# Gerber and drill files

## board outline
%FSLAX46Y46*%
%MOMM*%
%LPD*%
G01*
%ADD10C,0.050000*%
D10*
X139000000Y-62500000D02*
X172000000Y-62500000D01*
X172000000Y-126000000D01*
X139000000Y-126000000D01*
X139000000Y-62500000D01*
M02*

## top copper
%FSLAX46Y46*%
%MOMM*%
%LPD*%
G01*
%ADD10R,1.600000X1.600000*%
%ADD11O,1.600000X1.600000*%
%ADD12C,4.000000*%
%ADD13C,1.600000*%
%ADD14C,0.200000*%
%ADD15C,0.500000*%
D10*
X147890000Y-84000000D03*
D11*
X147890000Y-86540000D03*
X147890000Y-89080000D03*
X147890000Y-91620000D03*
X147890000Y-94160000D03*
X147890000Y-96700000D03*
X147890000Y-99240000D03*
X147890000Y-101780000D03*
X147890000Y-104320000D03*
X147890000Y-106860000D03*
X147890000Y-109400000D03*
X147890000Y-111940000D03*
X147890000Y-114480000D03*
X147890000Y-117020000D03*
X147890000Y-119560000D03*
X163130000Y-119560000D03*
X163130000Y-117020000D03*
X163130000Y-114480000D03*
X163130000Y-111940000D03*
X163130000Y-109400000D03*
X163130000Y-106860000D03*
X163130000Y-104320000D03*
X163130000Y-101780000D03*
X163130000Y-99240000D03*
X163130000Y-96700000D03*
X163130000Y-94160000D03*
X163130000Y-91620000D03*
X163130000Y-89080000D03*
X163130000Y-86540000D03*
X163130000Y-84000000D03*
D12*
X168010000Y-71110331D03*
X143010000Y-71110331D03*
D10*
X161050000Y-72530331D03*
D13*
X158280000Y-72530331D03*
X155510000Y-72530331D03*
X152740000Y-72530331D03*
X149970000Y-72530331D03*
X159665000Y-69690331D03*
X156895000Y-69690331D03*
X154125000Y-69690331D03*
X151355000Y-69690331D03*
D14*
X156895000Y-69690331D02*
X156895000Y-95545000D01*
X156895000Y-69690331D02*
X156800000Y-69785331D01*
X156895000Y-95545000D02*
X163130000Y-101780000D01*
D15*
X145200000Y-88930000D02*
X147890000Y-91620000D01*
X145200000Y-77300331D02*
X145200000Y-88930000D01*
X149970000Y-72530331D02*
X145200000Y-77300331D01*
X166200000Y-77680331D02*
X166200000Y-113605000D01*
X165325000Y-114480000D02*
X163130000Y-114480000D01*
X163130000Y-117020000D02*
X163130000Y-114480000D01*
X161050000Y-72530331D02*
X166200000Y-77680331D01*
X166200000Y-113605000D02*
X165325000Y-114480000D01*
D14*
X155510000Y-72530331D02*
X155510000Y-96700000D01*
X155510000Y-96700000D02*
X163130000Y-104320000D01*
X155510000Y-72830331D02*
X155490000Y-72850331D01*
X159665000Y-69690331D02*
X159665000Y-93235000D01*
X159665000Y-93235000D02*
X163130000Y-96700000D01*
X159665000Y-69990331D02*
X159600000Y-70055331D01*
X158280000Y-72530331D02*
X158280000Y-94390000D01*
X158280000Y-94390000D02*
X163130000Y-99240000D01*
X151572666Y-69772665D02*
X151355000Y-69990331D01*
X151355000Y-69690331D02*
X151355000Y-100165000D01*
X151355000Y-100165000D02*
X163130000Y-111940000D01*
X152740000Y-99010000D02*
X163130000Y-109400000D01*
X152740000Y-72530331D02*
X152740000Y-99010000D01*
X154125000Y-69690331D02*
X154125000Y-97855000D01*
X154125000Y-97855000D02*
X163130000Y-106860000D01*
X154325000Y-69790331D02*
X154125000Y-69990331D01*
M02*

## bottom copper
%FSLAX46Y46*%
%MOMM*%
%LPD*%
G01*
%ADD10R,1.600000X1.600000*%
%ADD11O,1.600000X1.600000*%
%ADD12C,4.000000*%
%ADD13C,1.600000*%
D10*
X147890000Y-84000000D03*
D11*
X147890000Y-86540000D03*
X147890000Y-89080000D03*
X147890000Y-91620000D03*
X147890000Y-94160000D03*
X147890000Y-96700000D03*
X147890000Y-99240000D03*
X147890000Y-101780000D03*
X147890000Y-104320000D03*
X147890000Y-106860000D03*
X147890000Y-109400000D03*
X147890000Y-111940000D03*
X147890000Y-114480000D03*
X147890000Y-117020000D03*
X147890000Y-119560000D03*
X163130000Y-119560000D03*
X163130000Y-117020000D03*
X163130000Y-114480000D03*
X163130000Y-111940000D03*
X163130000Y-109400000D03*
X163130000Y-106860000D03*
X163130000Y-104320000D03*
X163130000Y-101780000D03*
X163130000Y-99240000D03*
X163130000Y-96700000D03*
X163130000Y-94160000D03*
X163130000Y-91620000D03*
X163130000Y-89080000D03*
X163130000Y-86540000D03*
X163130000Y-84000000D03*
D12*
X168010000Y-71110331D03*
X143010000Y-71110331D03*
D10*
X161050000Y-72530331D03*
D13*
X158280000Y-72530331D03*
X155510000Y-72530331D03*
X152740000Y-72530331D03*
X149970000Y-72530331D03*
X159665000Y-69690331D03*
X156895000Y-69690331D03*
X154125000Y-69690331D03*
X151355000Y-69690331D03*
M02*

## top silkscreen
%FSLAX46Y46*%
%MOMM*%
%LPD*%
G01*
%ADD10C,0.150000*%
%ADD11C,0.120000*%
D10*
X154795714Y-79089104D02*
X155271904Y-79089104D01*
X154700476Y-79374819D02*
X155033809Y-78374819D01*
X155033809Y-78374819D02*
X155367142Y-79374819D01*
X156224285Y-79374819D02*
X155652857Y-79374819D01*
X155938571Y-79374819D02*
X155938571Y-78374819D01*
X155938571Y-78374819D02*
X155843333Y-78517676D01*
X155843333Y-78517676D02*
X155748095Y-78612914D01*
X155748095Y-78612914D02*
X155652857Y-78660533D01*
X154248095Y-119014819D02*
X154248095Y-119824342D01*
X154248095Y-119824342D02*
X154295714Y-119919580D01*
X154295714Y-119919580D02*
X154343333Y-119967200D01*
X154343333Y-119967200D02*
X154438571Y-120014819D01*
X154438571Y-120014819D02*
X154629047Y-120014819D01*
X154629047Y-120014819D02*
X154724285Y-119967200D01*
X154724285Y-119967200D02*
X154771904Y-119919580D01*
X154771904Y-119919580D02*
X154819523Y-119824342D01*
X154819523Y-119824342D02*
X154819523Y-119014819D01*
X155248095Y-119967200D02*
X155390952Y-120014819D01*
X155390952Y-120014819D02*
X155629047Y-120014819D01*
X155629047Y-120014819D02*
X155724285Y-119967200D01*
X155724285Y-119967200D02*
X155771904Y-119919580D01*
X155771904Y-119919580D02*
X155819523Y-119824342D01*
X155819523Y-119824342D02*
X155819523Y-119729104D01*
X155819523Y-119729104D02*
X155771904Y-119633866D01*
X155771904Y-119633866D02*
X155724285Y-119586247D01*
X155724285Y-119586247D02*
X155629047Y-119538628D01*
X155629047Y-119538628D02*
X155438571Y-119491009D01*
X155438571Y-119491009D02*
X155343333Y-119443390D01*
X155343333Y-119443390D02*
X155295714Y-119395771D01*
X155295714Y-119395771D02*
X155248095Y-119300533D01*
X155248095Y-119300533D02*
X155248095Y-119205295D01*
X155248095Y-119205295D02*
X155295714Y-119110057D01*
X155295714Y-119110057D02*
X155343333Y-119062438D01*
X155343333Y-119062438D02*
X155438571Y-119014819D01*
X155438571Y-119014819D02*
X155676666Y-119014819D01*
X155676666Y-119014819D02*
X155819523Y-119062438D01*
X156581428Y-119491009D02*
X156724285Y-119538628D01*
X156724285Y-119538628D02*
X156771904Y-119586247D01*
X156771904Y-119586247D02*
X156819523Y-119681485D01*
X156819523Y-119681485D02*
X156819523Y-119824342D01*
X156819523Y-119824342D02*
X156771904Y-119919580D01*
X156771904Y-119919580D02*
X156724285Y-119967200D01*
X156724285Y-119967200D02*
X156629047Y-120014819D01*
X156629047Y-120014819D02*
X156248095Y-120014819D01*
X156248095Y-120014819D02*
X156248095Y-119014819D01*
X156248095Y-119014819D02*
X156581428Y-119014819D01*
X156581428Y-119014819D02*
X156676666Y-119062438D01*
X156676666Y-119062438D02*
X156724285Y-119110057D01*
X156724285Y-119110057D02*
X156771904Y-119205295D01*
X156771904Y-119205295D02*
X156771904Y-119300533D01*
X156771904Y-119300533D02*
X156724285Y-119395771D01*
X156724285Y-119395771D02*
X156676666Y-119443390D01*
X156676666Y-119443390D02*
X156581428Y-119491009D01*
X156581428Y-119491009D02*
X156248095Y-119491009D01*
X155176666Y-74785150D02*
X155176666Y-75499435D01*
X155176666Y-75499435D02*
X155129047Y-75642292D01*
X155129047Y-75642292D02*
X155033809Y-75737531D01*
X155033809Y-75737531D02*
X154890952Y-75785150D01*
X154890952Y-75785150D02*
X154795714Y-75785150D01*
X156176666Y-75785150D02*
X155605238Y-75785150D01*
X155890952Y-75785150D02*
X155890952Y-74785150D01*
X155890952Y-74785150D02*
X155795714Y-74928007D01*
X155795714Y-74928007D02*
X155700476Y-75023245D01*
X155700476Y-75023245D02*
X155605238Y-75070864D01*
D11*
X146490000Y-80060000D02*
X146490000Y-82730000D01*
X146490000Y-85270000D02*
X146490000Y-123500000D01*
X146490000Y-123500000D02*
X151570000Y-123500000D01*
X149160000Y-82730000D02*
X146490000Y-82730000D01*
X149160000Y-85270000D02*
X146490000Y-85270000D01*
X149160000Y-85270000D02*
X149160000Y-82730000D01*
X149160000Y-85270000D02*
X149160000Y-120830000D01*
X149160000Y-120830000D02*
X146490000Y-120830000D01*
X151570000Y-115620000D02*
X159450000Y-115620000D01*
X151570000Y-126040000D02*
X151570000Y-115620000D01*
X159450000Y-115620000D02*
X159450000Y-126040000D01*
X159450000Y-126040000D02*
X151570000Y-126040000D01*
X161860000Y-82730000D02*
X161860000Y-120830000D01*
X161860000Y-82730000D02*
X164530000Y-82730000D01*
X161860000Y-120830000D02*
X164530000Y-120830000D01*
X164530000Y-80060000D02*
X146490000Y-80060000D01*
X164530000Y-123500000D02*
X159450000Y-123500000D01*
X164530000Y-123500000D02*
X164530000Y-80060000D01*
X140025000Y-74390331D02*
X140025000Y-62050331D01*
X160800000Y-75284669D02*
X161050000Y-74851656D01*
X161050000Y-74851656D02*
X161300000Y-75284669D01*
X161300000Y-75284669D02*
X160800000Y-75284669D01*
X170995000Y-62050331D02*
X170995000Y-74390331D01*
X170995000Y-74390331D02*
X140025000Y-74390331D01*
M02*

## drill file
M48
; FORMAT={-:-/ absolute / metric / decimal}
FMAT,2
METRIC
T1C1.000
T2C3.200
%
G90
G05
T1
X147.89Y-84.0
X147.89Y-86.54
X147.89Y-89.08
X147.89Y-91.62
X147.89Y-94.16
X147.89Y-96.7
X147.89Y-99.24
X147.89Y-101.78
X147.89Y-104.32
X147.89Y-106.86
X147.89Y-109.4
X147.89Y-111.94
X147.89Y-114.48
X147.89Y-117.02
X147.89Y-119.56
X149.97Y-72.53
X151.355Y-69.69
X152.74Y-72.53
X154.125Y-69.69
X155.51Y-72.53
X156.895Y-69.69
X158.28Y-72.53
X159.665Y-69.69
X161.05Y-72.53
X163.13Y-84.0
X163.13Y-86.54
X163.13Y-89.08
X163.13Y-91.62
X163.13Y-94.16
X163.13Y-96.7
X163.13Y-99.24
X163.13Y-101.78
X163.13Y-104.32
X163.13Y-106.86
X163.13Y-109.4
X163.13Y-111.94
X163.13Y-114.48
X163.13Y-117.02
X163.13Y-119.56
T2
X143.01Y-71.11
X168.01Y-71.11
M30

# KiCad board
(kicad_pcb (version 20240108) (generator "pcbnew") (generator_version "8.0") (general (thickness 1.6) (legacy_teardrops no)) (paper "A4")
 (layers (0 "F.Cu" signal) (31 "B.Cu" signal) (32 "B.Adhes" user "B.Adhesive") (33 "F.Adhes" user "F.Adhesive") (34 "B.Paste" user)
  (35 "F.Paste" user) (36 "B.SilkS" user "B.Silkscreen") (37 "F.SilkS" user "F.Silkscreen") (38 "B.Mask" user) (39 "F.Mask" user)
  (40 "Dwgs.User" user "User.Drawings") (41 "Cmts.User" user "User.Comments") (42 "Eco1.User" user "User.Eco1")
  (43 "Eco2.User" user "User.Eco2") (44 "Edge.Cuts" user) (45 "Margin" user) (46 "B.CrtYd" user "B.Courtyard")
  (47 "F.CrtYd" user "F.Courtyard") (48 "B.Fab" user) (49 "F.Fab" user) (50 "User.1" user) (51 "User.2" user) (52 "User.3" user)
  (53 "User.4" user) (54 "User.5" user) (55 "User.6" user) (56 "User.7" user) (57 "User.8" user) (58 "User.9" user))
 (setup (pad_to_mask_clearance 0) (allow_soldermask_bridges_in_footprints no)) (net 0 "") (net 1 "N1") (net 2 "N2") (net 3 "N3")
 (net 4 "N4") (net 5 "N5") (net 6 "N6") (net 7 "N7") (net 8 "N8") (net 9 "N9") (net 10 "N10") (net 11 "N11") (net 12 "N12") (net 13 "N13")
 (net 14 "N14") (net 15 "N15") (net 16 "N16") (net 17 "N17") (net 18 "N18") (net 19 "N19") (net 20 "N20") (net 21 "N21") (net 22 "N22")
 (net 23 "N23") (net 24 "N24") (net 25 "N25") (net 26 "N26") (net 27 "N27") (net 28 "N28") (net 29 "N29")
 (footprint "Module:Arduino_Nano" (layer "F.Cu") (at 147.89 84)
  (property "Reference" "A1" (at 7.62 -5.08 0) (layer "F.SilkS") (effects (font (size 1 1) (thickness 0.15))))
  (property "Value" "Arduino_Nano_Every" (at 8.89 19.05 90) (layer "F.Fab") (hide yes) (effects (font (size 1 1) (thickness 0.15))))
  (fp_line (start -1.4 -3.94) (end -1.4 -1.27) (stroke (width 0.12) (type solid)) (layer "F.SilkS"))
  (fp_line (start -1.4 1.27) (end -1.4 39.5) (stroke (width 0.12) (type solid)) (layer "F.SilkS"))
  (fp_line (start -1.4 39.5) (end 3.68 39.5) (stroke (width 0.12) (type solid)) (layer "F.SilkS"))
  (fp_line (start 1.27 -1.27) (end -1.4 -1.27) (stroke (width 0.12) (type solid)) (layer "F.SilkS"))
  (fp_line (start 1.27 1.27) (end -1.4 1.27) (stroke (width 0.12) (type solid)) (layer "F.SilkS"))
  (fp_line (start 1.27 1.27) (end 1.27 -1.27) (stroke (width 0.12) (type solid)) (layer "F.SilkS"))
  (fp_line (start 1.27 1.27) (end 1.27 36.83) (stroke (width 0.12) (type solid)) (layer "F.SilkS"))
  (fp_line (start 1.27 36.83) (end -1.4 36.83) (stroke (width 0.12) (type solid)) (layer "F.SilkS"))
  (fp_line (start 3.68 31.62) (end 11.56 31.62) (stroke (width 0.12) (type solid)) (layer "F.SilkS"))
  (fp_line (start 3.68 42.04) (end 3.68 31.62) (stroke (width 0.12) (type solid)) (layer "F.SilkS"))
  (fp_line (start 11.56 31.62) (end 11.56 42.04) (stroke (width 0.12) (type solid)) (layer "F.SilkS"))
  (fp_line (start 11.56 42.04) (end 3.68 42.04) (stroke (width 0.12) (type solid)) (layer "F.SilkS"))
  (fp_line (start 13.97 -1.27) (end 13.97 36.83) (stroke (width 0.12) (type solid)) (layer "F.SilkS"))
  (fp_line (start 13.97 -1.27) (end 16.64 -1.27) (stroke (width 0.12) (type solid)) (layer "F.SilkS"))
  (fp_line (start 13.97 36.83) (end 16.64 36.83) (stroke (width 0.12) (type solid)) (layer "F.SilkS"))
  (fp_line (start 16.64 -3.94) (end -1.4 -3.94) (stroke (width 0.12) (type solid)) (layer "F.SilkS"))
  (fp_line (start 16.64 39.5) (end 11.56 39.5) (stroke (width 0.12) (type solid)) (layer "F.SilkS"))
  (fp_line (start 16.64 39.5) (end 16.64 -3.94) (stroke (width 0.12) (type solid)) (layer "F.SilkS"))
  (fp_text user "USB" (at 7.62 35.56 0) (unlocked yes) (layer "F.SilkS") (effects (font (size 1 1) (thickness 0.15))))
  (pad "1" thru_hole rect (at 0 0) (size 1.6 1.6) (drill 1) (layers "*.Cu" "*.Mask") (remove_unused_layers no) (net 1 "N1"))
  (pad "2" thru_hole oval (at 0 2.54) (size 1.6 1.6) (drill 1) (layers "*.Cu" "*.Mask") (remove_unused_layers no) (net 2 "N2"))
  (pad "3" thru_hole oval (at 0 5.08) (size 1.6 1.6) (drill 1) (layers "*.Cu" "*.Mask") (remove_unused_layers no) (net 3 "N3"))
  (pad "4" thru_hole oval (at 0 7.62) (size 1.6 1.6) (drill 1) (layers "*.Cu" "*.Mask") (remove_unused_layers no) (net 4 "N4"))
  (pad "5" thru_hole oval (at 0 10.16) (size 1.6 1.6) (drill 1) (layers "*.Cu" "*.Mask") (remove_unused_layers no) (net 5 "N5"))
  (pad "6" thru_hole oval (at 0 12.7) (size 1.6 1.6) (drill 1) (layers "*.Cu" "*.Mask") (remove_unused_layers no) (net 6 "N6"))
  (pad "7" thru_hole oval (at 0 15.24) (size 1.6 1.6) (drill 1) (layers "*.Cu" "*.Mask") (remove_unused_layers no) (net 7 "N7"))
  (pad "8" thru_hole oval (at 0 17.78) (size 1.6 1.6) (drill 1) (layers "*.Cu" "*.Mask") (remove_unused_layers no) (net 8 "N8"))
  (pad "9" thru_hole oval (at 0 20.32) (size 1.6 1.6) (drill 1) (layers "*.Cu" "*.Mask") (remove_unused_layers no) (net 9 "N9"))
  (pad "10" thru_hole oval (at 0 22.86) (size 1.6 1.6) (drill 1) (layers "*.Cu" "*.Mask") (remove_unused_layers no) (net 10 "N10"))
  (pad "11" thru_hole oval (at 0 25.4) (size 1.6 1.6) (drill 1) (layers "*.Cu" "*.Mask") (remove_unused_layers no) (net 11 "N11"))
  (pad "12" thru_hole oval (at 0 27.94) (size 1.6 1.6) (drill 1) (layers "*.Cu" "*.Mask") (remove_unused_layers no) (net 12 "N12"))
  (pad "13" thru_hole oval (at 0 30.48) (size 1.6 1.6) (drill 1) (layers "*.Cu" "*.Mask") (remove_unused_layers no) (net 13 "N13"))
  (pad "14" thru_hole oval (at 0 33.02) (size 1.6 1.6) (drill 1) (layers "*.Cu" "*.Mask") (remove_unused_layers no) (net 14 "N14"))
  (pad "15" thru_hole oval (at 0 35.56) (size 1.6 1.6) (drill 1) (layers "*.Cu" "*.Mask") (remove_unused_layers no) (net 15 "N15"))
  (pad "16" thru_hole oval (at 15.24 35.56) (size 1.6 1.6) (drill 1) (layers "*.Cu" "*.Mask") (remove_unused_layers no) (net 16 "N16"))
  (pad "17" thru_hole oval (at 15.24 33.02) (size 1.6 1.6) (drill 1) (layers "*.Cu" "*.Mask") (remove_unused_layers no) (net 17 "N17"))
  (pad "18" thru_hole oval (at 15.24 30.48) (size 1.6 1.6) (drill 1) (layers "*.Cu" "*.Mask") (remove_unused_layers no) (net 17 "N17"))
  (pad "19" thru_hole oval (at 15.24 27.94) (size 1.6 1.6) (drill 1) (layers "*.Cu" "*.Mask") (remove_unused_layers no) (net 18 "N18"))
  (pad "20" thru_hole oval (at 15.24 25.4) (size 1.6 1.6) (drill 1) (layers "*.Cu" "*.Mask") (remove_unused_layers no) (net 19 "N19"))
  (pad "21" thru_hole oval (at 15.24 22.86) (size 1.6 1.6) (drill 1) (layers "*.Cu" "*.Mask") (remove_unused_layers no) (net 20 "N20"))
  (pad "22" thru_hole oval (at 15.24 20.32) (size 1.6 1.6) (drill 1) (layers "*.Cu" "*.Mask") (remove_unused_layers no) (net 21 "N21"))
  (pad "23" thru_hole oval (at 15.24 17.78) (size 1.6 1.6) (drill 1) (layers "*.Cu" "*.Mask") (remove_unused_layers no) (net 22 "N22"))
  (pad "24" thru_hole oval (at 15.24 15.24) (size 1.6 1.6) (drill 1) (layers "*.Cu" "*.Mask") (remove_unused_layers no) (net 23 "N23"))
  (pad "25" thru_hole oval (at 15.24 12.7) (size 1.6 1.6) (drill 1) (layers "*.Cu" "*.Mask") (remove_unused_layers no) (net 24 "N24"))
  (pad "26" thru_hole oval (at 15.24 10.16) (size 1.6 1.6) (drill 1) (layers "*.Cu" "*.Mask") (remove_unused_layers no) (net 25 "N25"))
  (pad "27" thru_hole oval (at 15.24 7.62) (size 1.6 1.6) (drill 1) (layers "*.Cu" "*.Mask") (remove_unused_layers no) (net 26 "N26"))
  (pad "28" thru_hole oval (at 15.24 5.08) (size 1.6 1.6) (drill 1) (layers "*.Cu" "*.Mask") (remove_unused_layers no) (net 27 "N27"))
  (pad "29" thru_hole oval (at 15.24 2.54) (size 1.6 1.6) (drill 1) (layers "*.Cu" "*.Mask") (remove_unused_layers no) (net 4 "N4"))
  (pad "30" thru_hole oval (at 15.24 0) (size 1.6 1.6) (drill 1) (layers "*.Cu" "*.Mask") (remove_unused_layers no) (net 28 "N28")))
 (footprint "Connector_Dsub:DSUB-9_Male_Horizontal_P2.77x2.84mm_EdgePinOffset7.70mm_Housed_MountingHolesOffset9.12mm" (layer "F.Cu")
  (at 161.05 72.530331 180)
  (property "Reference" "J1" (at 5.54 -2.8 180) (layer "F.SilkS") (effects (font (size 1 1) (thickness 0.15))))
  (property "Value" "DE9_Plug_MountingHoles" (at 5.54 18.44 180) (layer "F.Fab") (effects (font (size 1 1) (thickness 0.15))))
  (fp_line (start 21.025 -1.86) (end 21.025 10.48) (stroke (width 0.12) (type solid)) (layer "F.SilkS"))
  (fp_line (start 0.25 -2.754338) (end 0 -2.321325) (stroke (width 0.12) (type solid)) (layer "F.SilkS"))
  (fp_line (start 0 -2.321325) (end -0.25 -2.754338) (stroke (width 0.12) (type solid)) (layer "F.SilkS"))
  (fp_line (start -0.25 -2.754338) (end 0.25 -2.754338) (stroke (width 0.12) (type solid)) (layer "F.SilkS"))
  (fp_line (start -9.945 10.48) (end -9.945 -1.86) (stroke (width 0.12) (type solid)) (layer "F.SilkS"))
  (fp_line (start -9.945 -1.86) (end 21.025 -1.86) (stroke (width 0.12) (type solid)) (layer "F.SilkS"))
  (pad "0" thru_hole circle (at -6.96 1.42 180) (size 4 4) (drill 3.2) (layers "*.Cu" "*.Mask") (remove_unused_layers no) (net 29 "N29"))
  (pad "0" thru_hole circle (at 18.04 1.42 180) (size 4 4) (drill 3.2) (layers "*.Cu" "*.Mask") (remove_unused_layers no) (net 29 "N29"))
  (pad "1" thru_hole rect (at 0 0 180) (size 1.6 1.6) (drill 1) (layers "*.Cu" "*.Mask") (remove_unused_layers no) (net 17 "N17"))
  (pad "2" thru_hole circle (at 2.77 0 180) (size 1.6 1.6) (drill 1) (layers "*.Cu" "*.Mask") (remove_unused_layers no) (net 23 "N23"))
  (pad "3" thru_hole circle (at 5.54 0 180) (size 1.6 1.6) (drill 1) (layers "*.Cu" "*.Mask") (remove_unused_layers no) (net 21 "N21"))
  (pad "4" thru_hole circle (at 8.31 0 180) (size 1.6 1.6) (drill 1) (layers "*.Cu" "*.Mask") (remove_unused_layers no) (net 19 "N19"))
  (pad "5" thru_hole circle (at 11.08 0 180) (size 1.6 1.6) (drill 1) (layers "*.Cu" "*.Mask") (remove_unused_layers no) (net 4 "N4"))
  (pad "6" thru_hole circle (at 1.385 2.84 180) (size 1.6 1.6) (drill 1) (layers "*.Cu" "*.Mask") (remove_unused_layers no) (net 24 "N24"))
  (pad "7" thru_hole circle (at 4.155 2.84 180) (size 1.6 1.6) (drill 1) (layers "*.Cu" "*.Mask") (remove_unused_layers no) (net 22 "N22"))
  (pad "8" thru_hole circle (at 6.925 2.84 180) (size 1.6 1.6) (drill 1) (layers "*.Cu" "*.Mask") (remove_unused_layers no) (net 20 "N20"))
  (pad "9" thru_hole circle (at 9.695 2.84 180) (size 1.6 1.6) (drill 1) (layers "*.Cu" "*.Mask") (remove_unused_layers no) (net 18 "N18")))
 (gr_rect (start 139 62.5) (end 172 126) (stroke (width 0.05) (type default)) (fill none) (layer "Edge.Cuts"))
 (segment (start 156.895 69.690331) (end 156.895 95.545) (width 0.2) (layer "F.Cu") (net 22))
 (segment (start 156.895 69.690331) (end 156.8 69.785331) (width 0.2) (layer "F.Cu") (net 22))
 (segment (start 156.895 95.545) (end 163.13 101.78) (width 0.2) (layer "F.Cu") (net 22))
 (segment (start 145.2 88.93) (end 147.89 91.62) (width 0.5) (layer "F.Cu") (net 4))
 (segment (start 145.2 77.300331) (end 145.2 88.93) (width 0.5) (layer "F.Cu") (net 4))
 (segment (start 149.97 72.530331) (end 145.2 77.300331) (width 0.5) (layer "F.Cu") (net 4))
 (segment (start 166.2 77.680331) (end 166.2 113.605) (width 0.5) (layer "F.Cu") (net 17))
 (segment (start 165.325 114.48) (end 163.13 114.48) (width 0.5) (layer "F.Cu") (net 17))
 (segment (start 163.13 117.02) (end 163.13 114.48) (width 0.5) (layer "F.Cu") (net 17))
 (segment (start 161.05 72.530331) (end 166.2 77.680331) (width 0.5) (layer "F.Cu") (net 17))
 (segment (start 166.2 113.605) (end 165.325 114.48) (width 0.5) (layer "F.Cu") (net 17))
 (segment (start 155.51 72.530331) (end 155.51 96.7) (width 0.2) (layer "F.Cu") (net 21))
 (segment (start 155.51 96.7) (end 163.13 104.32) (width 0.2) (layer "F.Cu") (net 21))
 (segment (start 155.51 72.830331) (end 155.49 72.850331) (width 0.2) (layer "F.Cu") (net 21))
 (segment (start 159.665 69.690331) (end 159.665 93.235) (width 0.2) (layer "F.Cu") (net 24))
 (segment (start 159.665 93.235) (end 163.13 96.7) (width 0.2) (layer "F.Cu") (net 24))
 (segment (start 159.665 69.990331) (end 159.6 70.055331) (width 0.2) (layer "F.Cu") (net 24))
 (segment (start 158.28 72.530331) (end 158.28 94.39) (width 0.2) (layer "F.Cu") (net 23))
 (segment (start 158.28 94.39) (end 163.13 99.24) (width 0.2) (layer "F.Cu") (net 23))
 (segment (start 151.572666 69.772665) (end 151.355 69.990331) (width 0.2) (layer "F.Cu") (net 18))
 (segment (start 151.355 69.690331) (end 151.355 100.165) (width 0.2) (layer "F.Cu") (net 18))
 (segment (start 151.355 100.165) (end 163.13 111.94) (width 0.2) (layer "F.Cu") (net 18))
 (segment (start 152.74 99.01) (end 163.13 109.4) (width 0.2) (layer "F.Cu") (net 19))
 (segment (start 152.74 72.530331) (end 152.74 99.01) (width 0.2) (layer "F.Cu") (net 19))
 (segment (start 154.125 69.690331) (end 154.125 97.855) (width 0.2) (layer "F.Cu") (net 20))
 (segment (start 154.125 97.855) (end 163.13 106.86) (width 0.2) (layer "F.Cu") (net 20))
 (segment (start 154.325 69.790331) (end 154.125 69.990331) (width 0.2) (layer "F.Cu") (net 20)))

